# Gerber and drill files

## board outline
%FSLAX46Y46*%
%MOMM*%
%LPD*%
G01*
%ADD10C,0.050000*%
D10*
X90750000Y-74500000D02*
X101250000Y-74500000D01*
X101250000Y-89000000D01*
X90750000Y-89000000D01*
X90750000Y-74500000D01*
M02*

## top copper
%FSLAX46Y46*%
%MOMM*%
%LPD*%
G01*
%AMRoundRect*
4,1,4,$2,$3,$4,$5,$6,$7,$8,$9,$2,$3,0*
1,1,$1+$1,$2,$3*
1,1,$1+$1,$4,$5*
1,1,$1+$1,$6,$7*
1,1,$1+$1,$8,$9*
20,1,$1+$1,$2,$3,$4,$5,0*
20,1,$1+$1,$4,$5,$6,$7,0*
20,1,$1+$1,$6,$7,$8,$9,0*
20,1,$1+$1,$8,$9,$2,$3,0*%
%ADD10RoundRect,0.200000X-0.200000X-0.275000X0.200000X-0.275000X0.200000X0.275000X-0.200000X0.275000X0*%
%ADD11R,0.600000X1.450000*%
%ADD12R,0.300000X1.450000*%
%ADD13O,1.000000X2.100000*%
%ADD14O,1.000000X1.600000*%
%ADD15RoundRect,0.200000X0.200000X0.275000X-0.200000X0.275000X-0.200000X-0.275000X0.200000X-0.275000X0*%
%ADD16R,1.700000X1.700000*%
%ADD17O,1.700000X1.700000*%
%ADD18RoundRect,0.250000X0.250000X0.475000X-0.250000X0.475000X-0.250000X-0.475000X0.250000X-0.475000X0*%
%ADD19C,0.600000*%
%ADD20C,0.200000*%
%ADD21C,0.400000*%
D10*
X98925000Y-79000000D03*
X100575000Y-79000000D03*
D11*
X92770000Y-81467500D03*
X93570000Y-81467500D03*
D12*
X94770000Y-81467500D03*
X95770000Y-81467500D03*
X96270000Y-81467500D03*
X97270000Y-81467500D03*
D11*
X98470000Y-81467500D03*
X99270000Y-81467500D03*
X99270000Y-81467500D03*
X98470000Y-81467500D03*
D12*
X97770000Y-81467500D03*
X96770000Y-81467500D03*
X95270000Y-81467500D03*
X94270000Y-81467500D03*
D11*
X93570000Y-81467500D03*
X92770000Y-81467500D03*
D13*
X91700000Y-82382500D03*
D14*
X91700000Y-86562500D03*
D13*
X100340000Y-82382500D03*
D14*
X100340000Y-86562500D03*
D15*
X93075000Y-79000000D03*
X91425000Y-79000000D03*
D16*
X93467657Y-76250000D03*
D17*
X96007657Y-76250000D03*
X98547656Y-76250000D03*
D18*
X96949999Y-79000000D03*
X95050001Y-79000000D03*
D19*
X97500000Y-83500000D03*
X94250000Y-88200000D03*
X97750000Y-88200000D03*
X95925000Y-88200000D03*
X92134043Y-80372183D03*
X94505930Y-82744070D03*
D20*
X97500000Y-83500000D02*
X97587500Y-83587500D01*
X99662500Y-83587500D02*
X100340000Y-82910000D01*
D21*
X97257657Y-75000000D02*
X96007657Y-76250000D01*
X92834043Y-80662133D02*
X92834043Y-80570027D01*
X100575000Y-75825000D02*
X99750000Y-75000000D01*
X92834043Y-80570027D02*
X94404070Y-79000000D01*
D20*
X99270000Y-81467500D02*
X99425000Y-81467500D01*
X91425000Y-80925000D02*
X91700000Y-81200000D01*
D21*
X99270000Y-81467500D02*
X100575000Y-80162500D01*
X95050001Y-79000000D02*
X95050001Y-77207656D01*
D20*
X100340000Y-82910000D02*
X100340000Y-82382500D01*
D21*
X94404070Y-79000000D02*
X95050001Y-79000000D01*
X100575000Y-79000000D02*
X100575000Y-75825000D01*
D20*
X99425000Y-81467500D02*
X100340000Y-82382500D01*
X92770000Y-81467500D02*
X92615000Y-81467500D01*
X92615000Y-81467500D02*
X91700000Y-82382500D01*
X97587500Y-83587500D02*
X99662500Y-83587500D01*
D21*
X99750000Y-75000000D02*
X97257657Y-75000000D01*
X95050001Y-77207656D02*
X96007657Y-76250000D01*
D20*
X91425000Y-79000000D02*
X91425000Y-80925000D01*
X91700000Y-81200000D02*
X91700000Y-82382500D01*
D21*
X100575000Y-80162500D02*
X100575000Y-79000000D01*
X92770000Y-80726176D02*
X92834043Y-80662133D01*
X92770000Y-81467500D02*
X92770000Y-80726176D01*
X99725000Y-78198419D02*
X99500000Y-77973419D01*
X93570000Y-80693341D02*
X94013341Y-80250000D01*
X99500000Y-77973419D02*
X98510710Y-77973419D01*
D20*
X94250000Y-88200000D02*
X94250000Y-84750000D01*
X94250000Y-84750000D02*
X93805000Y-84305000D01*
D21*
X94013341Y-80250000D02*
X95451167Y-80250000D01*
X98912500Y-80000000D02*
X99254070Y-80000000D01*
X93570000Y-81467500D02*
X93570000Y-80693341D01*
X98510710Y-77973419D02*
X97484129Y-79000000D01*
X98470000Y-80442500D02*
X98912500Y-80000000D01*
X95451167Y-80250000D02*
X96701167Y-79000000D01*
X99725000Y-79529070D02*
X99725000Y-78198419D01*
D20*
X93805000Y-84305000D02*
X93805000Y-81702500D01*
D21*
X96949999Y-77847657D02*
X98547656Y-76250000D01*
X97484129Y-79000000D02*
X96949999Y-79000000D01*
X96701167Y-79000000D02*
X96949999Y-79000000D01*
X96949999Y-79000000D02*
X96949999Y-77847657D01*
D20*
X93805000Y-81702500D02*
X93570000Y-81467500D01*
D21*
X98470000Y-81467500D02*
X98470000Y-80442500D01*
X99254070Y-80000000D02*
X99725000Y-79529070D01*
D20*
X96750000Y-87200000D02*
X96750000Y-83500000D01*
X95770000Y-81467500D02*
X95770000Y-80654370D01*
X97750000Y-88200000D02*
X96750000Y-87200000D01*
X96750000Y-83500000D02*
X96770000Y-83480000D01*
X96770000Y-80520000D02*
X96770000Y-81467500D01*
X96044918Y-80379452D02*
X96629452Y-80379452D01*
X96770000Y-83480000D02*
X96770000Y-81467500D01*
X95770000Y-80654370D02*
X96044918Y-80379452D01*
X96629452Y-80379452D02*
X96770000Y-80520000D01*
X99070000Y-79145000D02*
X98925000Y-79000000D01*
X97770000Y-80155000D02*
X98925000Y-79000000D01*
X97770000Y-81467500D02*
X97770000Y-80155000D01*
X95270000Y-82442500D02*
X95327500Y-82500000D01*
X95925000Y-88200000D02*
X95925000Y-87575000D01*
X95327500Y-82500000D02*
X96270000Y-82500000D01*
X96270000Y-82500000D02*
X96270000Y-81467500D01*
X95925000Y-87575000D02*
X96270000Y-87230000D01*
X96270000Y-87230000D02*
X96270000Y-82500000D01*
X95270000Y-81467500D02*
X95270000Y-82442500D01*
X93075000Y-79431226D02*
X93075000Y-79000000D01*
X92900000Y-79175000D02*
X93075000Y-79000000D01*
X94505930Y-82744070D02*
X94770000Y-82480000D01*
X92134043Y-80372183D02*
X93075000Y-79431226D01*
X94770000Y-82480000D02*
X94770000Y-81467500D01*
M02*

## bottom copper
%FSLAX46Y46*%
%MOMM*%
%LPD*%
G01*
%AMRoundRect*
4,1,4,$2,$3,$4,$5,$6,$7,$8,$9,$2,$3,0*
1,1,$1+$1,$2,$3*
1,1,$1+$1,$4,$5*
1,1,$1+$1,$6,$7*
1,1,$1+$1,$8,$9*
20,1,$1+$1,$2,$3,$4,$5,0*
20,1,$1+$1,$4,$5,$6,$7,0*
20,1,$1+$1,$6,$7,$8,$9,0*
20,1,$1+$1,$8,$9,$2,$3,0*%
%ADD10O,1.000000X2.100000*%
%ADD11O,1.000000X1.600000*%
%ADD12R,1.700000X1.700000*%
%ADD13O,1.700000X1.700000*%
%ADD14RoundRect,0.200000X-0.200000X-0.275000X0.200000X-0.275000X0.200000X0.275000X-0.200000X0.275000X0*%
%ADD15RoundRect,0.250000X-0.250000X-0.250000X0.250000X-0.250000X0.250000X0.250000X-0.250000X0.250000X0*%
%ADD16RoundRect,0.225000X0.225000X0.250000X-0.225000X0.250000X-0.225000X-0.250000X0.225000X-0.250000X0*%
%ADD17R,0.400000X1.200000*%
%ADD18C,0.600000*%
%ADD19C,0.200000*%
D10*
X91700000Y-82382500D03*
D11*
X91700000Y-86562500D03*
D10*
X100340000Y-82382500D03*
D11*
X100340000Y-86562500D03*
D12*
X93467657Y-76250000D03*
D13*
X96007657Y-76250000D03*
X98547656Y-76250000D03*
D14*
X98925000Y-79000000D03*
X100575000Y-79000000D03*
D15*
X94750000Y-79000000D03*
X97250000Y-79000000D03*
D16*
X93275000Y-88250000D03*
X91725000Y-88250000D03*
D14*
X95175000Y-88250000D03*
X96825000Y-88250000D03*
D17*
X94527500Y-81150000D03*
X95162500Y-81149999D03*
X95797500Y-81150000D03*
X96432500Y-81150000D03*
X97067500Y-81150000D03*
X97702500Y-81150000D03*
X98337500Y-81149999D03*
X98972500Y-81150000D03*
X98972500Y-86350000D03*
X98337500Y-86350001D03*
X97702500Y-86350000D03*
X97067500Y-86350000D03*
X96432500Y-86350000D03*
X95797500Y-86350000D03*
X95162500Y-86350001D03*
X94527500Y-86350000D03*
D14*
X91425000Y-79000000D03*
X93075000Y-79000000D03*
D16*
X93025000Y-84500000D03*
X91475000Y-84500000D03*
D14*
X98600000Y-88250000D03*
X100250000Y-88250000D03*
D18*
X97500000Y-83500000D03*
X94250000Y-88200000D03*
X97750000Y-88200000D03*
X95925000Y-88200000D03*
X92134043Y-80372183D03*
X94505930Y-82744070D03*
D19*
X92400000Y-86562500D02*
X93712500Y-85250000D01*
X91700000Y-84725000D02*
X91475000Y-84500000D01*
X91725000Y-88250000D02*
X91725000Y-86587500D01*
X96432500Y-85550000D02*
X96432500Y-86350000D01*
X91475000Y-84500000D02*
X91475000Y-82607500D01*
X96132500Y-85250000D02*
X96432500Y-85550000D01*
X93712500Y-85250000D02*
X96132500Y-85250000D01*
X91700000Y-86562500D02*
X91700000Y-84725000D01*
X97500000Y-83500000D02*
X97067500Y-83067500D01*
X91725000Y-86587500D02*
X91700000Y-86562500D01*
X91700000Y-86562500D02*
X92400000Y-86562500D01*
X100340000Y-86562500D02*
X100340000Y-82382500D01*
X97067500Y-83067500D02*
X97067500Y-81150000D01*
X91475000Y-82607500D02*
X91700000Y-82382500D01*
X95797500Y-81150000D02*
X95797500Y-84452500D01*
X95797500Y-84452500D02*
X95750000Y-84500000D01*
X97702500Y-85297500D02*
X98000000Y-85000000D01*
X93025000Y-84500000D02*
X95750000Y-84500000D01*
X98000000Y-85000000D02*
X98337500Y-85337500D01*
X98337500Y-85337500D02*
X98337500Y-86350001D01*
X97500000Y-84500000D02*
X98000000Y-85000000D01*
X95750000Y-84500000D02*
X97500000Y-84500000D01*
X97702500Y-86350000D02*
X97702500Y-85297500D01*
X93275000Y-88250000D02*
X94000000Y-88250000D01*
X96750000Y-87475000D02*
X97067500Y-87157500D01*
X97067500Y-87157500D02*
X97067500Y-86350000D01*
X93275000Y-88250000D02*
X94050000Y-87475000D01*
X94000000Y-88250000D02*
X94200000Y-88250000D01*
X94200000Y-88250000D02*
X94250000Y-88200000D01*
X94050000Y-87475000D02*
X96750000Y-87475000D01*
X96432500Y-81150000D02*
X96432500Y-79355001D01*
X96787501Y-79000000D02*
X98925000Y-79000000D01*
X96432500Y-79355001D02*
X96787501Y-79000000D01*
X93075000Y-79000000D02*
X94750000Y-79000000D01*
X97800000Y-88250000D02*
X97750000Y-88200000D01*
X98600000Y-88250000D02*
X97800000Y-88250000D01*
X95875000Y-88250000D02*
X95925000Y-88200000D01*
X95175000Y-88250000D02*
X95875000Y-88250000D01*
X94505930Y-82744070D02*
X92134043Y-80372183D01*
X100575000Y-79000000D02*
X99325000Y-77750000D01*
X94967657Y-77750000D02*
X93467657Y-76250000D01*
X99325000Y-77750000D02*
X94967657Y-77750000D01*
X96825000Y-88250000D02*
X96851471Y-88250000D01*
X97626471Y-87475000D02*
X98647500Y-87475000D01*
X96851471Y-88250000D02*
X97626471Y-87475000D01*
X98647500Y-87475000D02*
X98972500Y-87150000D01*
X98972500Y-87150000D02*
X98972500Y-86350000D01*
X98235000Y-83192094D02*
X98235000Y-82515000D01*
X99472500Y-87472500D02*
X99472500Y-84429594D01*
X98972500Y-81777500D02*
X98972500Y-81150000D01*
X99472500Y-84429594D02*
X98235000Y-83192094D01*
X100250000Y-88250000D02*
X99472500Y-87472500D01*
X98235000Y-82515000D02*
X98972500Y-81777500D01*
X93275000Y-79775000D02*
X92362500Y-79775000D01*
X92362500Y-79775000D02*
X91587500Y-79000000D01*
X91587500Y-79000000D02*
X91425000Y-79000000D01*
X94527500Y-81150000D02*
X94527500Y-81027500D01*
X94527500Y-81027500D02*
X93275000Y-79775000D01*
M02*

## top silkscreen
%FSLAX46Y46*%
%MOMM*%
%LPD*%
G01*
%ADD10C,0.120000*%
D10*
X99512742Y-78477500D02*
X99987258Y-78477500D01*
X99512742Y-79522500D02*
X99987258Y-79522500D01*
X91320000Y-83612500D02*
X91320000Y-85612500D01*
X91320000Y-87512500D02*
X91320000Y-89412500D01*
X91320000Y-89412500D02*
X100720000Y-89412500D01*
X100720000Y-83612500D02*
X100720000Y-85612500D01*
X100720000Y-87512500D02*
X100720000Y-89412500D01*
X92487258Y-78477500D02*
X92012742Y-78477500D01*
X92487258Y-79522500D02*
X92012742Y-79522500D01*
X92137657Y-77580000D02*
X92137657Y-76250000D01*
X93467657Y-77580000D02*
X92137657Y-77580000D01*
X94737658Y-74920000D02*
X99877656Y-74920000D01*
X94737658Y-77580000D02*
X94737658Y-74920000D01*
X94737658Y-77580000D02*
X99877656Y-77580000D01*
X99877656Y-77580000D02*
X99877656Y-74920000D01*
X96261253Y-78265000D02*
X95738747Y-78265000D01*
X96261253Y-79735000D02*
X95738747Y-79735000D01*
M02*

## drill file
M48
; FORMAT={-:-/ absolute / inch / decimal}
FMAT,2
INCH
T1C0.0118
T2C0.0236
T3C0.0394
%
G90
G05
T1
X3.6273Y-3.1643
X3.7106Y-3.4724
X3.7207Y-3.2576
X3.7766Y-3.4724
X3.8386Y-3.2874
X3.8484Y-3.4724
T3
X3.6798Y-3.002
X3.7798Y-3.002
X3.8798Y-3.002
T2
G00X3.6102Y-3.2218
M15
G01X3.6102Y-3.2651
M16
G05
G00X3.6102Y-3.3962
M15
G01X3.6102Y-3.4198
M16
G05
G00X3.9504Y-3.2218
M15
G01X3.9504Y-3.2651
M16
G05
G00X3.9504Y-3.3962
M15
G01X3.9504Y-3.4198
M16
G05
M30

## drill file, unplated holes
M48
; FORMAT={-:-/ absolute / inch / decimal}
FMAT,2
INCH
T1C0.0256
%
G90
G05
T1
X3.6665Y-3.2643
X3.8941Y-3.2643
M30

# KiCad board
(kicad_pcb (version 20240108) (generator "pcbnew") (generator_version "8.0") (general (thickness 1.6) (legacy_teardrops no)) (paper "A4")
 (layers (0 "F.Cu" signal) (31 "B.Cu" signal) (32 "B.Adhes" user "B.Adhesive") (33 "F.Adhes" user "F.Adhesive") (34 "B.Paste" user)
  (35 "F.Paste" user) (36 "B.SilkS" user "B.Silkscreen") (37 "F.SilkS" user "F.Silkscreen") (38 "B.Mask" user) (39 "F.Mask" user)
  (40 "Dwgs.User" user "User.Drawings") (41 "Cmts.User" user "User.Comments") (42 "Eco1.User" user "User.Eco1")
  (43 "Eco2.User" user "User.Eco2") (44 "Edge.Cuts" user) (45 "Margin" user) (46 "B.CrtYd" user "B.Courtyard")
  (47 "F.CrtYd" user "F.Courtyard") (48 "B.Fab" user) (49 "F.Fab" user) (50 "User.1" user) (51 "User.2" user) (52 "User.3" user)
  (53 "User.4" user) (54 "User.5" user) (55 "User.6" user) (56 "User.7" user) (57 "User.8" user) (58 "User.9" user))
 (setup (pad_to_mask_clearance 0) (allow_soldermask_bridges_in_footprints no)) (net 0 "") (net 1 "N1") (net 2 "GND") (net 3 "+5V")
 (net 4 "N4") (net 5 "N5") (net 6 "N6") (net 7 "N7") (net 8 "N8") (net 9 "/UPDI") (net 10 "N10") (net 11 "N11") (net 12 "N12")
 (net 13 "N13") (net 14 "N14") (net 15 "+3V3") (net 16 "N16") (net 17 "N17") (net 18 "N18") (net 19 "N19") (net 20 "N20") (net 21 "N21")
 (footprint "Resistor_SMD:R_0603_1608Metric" (layer "F.Cu") (at 99.75 79)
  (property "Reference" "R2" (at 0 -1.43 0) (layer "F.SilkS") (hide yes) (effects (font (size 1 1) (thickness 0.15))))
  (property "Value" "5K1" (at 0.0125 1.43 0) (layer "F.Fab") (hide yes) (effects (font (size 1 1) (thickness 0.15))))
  (fp_line (start -0.237258 -0.5225) (end 0.237258 -0.5225) (stroke (width 0.12) (type solid)) (layer "F.SilkS"))
  (fp_line (start -0.237258 0.5225) (end 0.237258 0.5225) (stroke (width 0.12) (type solid)) (layer "F.SilkS"))
  (pad "1" smd roundrect (at -0.825 0) (size 0.8 0.95) (layers "F.Cu" "F.Paste" "F.Mask") (roundrect_rratio 0.25) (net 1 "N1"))
  (pad "2" smd roundrect (at 0.825 0) (size 0.8 0.95) (layers "F.Cu" "F.Paste" "F.Mask") (roundrect_rratio 0.25) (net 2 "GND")))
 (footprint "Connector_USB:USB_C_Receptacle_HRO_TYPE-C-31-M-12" (layer "F.Cu") (at 96.02 85.5125)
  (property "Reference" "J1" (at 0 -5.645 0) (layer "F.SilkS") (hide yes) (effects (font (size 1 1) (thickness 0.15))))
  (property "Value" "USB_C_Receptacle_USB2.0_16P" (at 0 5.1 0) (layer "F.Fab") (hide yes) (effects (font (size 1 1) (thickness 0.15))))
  (fp_line (start -4.7 -1.9) (end -4.7 0.1) (stroke (width 0.12) (type solid)) (layer "F.SilkS"))
  (fp_line (start -4.7 2) (end -4.7 3.9) (stroke (width 0.12) (type solid)) (layer "F.SilkS"))
  (fp_line (start -4.7 3.9) (end 4.7 3.9) (stroke (width 0.12) (type solid)) (layer "F.SilkS"))
  (fp_line (start 4.7 -1.9) (end 4.7 0.1) (stroke (width 0.12) (type solid)) (layer "F.SilkS"))
  (fp_line (start 4.7 2) (end 4.7 3.9) (stroke (width 0.12) (type solid)) (layer "F.SilkS"))
  (pad "" np_thru_hole circle (at -2.89 -2.6) (size 0.65 0.65) (drill 0.65) (layers "*.Cu" "*.Mask"))
  (pad "" np_thru_hole circle (at 2.89 -2.6) (size 0.65 0.65) (drill 0.65) (layers "*.Cu" "*.Mask"))
  (pad "A1" smd rect (at -3.25 -4.045) (size 0.6 1.45) (layers "F.Cu" "F.Paste" "F.Mask") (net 2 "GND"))
  (pad "A4" smd rect (at -2.45 -4.045) (size 0.6 1.45) (layers "F.Cu" "F.Paste" "F.Mask") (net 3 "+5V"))
  (pad "A5" smd rect (at -1.25 -4.045) (size 0.3 1.45) (layers "F.Cu" "F.Paste" "F.Mask") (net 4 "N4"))
  (pad "A6" smd rect (at -0.25 -4.045) (size 0.3 1.45) (layers "F.Cu" "F.Paste" "F.Mask") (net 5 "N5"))
  (pad "A7" smd rect (at 0.25 -4.045) (size 0.3 1.45) (layers "F.Cu" "F.Paste" "F.Mask") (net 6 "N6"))
  (pad "A8" smd rect (at 1.25 -4.045) (size 0.3 1.45) (layers "F.Cu" "F.Paste" "F.Mask") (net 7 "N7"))
  (pad "A9" smd rect (at 2.45 -4.045) (size 0.6 1.45) (layers "F.Cu" "F.Paste" "F.Mask") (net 3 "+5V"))
  (pad "A12" smd rect (at 3.25 -4.045) (size 0.6 1.45) (layers "F.Cu" "F.Paste" "F.Mask") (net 2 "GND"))
  (pad "B1" smd rect (at 3.25 -4.045) (size 0.6 1.45) (layers "F.Cu" "F.Paste" "F.Mask") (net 2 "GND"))
  (pad "B4" smd rect (at 2.45 -4.045) (size 0.6 1.45) (layers "F.Cu" "F.Paste" "F.Mask") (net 3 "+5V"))
  (pad "B5" smd rect (at 1.75 -4.045) (size 0.3 1.45) (layers "F.Cu" "F.Paste" "F.Mask") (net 1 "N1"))
  (pad "B6" smd rect (at 0.75 -4.045) (size 0.3 1.45) (layers "F.Cu" "F.Paste" "F.Mask") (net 5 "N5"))
  (pad "B7" smd rect (at -0.75 -4.045) (size 0.3 1.45) (layers "F.Cu" "F.Paste" "F.Mask") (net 6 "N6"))
  (pad "B8" smd rect (at -1.75 -4.045) (size 0.3 1.45) (layers "F.Cu" "F.Paste" "F.Mask") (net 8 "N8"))
  (pad "B9" smd rect (at -2.45 -4.045) (size 0.6 1.45) (layers "F.Cu" "F.Paste" "F.Mask") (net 3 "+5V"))
  (pad "B12" smd rect (at -3.25 -4.045) (size 0.6 1.45) (layers "F.Cu" "F.Paste" "F.Mask") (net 2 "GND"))
  (pad "S1" thru_hole oval (at -4.32 -3.13) (size 1 2.1) (drill oval 0.6 1.7) (layers "*.Cu" "*.Mask") (remove_unused_layers no)
   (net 2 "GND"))
  (pad "S1" thru_hole oval (at -4.32 1.05) (size 1 1.6) (drill oval 0.6 1.2) (layers "*.Cu" "*.Mask") (remove_unused_layers no)
   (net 2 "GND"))
  (pad "S1" thru_hole oval (at 4.32 -3.13) (size 1 2.1) (drill oval 0.6 1.7) (layers "*.Cu" "*.Mask") (remove_unused_layers no)
   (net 2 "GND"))
  (pad "S1" thru_hole oval (at 4.32 1.05) (size 1 1.6) (drill oval 0.6 1.2) (layers "*.Cu" "*.Mask") (remove_unused_layers no) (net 2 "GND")))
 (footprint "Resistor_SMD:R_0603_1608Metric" (layer "F.Cu") (at 92.25 79 180)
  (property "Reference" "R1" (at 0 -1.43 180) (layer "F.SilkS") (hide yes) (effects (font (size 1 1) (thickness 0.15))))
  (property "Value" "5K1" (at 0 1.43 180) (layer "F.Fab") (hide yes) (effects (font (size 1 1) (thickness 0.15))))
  (fp_line (start -0.237258 0.5225) (end 0.237258 0.5225) (stroke (width 0.12) (type solid)) (layer "F.SilkS"))
  (fp_line (start -0.237258 -0.5225) (end 0.237258 -0.5225) (stroke (width 0.12) (type solid)) (layer "F.SilkS"))
  (pad "1" smd roundrect (at -0.825 0 180) (size 0.8 0.95) (layers "F.Cu" "F.Paste" "F.Mask") (roundrect_rratio 0.25) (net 4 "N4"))
  (pad "2" smd roundrect (at 0.825 0 180) (size 0.8 0.95) (layers "F.Cu" "F.Paste" "F.Mask") (roundrect_rratio 0.25) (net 2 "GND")))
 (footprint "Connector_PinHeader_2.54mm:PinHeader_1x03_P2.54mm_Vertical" (layer "F.Cu") (at 93.467657 76.25 90)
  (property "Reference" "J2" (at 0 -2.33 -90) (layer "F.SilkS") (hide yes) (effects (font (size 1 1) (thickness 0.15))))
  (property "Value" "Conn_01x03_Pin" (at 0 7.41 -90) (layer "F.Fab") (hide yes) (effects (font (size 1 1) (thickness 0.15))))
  (fp_line (start -1.33 -1.33) (end 0 -1.33) (stroke (width 0.12) (type solid)) (layer "F.SilkS"))
  (fp_line (start -1.33 0) (end -1.33 -1.33) (stroke (width 0.12) (type solid)) (layer "F.SilkS"))
  (fp_line (start 1.33 1.270001) (end 1.33 6.409999) (stroke (width 0.12) (type solid)) (layer "F.SilkS"))
  (fp_line (start -1.33 1.270001) (end 1.33 1.270001) (stroke (width 0.12) (type solid)) (layer "F.SilkS"))
  (fp_line (start -1.33 1.270001) (end -1.33 6.409999) (stroke (width 0.12) (type solid)) (layer "F.SilkS"))
  (fp_line (start -1.33 6.409999) (end 1.33 6.409999) (stroke (width 0.12) (type solid)) (layer "F.SilkS"))
  (pad "1" thru_hole rect (at 0 0 90) (size 1.7 1.7) (drill 1) (layers "*.Cu" "*.Mask") (remove_unused_layers no) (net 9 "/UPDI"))
  (pad "2" thru_hole oval (at 0 2.54 90) (size 1.7 1.7) (drill 1) (layers "*.Cu" "*.Mask") (remove_unused_layers no) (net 2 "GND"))
  (pad "3" thru_hole oval (at 0 5.079999 90) (size 1.7 1.7) (drill 1) (layers "*.Cu" "*.Mask") (remove_unused_layers no) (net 3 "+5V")))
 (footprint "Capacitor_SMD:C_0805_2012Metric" (layer "F.Cu") (at 96 79 180)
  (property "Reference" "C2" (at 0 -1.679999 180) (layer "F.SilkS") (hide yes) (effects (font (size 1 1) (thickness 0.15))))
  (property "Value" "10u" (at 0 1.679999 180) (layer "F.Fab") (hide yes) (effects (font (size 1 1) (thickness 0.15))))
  (fp_line (start -0.261253 0.735) (end 0.261253 0.735) (stroke (width 0.12) (type solid)) (layer "F.SilkS"))
  (fp_line (start -0.261253 -0.735) (end 0.261253 -0.735) (stroke (width 0.12) (type solid)) (layer "F.SilkS"))
  (pad "1" smd roundrect (at -0.949999 0 180) (size 1 1.45) (layers "F.Cu" "F.Paste" "F.Mask") (roundrect_rratio 0.25) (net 3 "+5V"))
  (pad "2" smd roundrect (at 0.949999 0 180) (size 1 1.45) (layers "F.Cu" "F.Paste" "F.Mask") (roundrect_rratio 0.25) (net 2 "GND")))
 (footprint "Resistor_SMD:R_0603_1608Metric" (layer "B.Cu") (at 99.75 79)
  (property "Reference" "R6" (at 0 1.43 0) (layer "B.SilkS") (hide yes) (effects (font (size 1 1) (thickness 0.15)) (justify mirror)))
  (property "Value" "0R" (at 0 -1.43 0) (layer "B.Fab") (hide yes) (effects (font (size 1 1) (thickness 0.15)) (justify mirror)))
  (pad "1" smd roundrect (at -0.825 0) (size 0.8 0.95) (layers "B.Cu" "B.Paste" "B.Mask") (roundrect_rratio 0.25) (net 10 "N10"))
  (pad "2" smd roundrect (at 0.825 0) (size 0.8 0.95) (layers "B.Cu" "B.Paste" "B.Mask") (roundrect_rratio 0.25) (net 9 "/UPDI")))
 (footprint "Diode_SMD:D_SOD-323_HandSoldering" (layer "B.Cu") (at 96 79)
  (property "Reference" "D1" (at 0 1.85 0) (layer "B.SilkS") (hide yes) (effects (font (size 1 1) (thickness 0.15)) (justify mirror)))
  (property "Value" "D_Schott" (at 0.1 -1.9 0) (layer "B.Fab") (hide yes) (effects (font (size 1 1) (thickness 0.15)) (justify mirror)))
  (pad "1" smd roundrect (at -1.25 0) (size 1 1) (layers "B.Cu" "B.Paste" "B.Mask") (roundrect_rratio 0.25) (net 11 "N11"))
  (pad "2" smd roundrect (at 1.25 0) (size 1 1) (layers "B.Cu" "B.Paste" "B.Mask") (roundrect_rratio 0.25) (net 10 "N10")))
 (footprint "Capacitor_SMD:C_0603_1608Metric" (layer "B.Cu") (at 92.5 88.25 180)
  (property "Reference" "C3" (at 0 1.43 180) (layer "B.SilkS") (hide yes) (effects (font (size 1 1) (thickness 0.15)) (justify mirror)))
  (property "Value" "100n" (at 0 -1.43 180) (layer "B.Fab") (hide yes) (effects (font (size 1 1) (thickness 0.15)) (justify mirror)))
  (pad "1" smd roundrect (at -0.775 0 180) (size 0.9 0.95) (layers "B.Cu" "B.Paste" "B.Mask") (roundrect_rratio 0.25) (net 3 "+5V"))
  (pad "2" smd roundrect (at 0.775 0 180) (size 0.9 0.95) (layers "B.Cu" "B.Paste" "B.Mask") (roundrect_rratio 0.25) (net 2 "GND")))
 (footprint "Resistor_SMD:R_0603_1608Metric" (layer "B.Cu") (at 96 88.25)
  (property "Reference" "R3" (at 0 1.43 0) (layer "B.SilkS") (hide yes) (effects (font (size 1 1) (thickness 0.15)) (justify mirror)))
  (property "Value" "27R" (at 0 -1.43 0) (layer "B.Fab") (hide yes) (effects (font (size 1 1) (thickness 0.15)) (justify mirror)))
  (pad "1" smd roundrect (at -0.825 0) (size 0.8 0.95) (layers "B.Cu" "B.Paste" "B.Mask") (roundrect_rratio 0.25) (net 6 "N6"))
  (pad "2" smd roundrect (at 0.825 0) (size 0.8 0.95) (layers "B.Cu" "B.Paste" "B.Mask") (roundrect_rratio 0.25) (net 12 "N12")))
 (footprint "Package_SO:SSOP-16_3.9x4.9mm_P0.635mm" (layer "B.Cu") (at 96.75 83.75 -90)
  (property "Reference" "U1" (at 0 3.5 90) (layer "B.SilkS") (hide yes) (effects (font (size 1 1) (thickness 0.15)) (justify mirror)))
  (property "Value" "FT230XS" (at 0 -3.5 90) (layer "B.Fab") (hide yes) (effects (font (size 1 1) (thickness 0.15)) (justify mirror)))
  (pad "1" smd rect (at -2.6 2.2225 270) (size 1.2 0.4) (layers "B.Cu" "B.Paste" "B.Mask") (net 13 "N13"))
  (pad "2" smd rect (at -2.600001 1.5875 270) (size 1.2 0.4) (layers "B.Cu" "B.Paste" "B.Mask") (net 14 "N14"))
  (pad "3" smd rect (at -2.6 0.9525 270) (size 1.2 0.4) (layers "B.Cu" "B.Paste" "B.Mask") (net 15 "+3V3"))
  (pad "4" smd rect (at -2.6 0.3175 270) (size 1.2 0.4) (layers "B.Cu" "B.Paste" "B.Mask") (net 10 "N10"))
  (pad "5" smd rect (at -2.6 -0.3175 270) (size 1.2 0.4) (layers "B.Cu" "B.Paste" "B.Mask") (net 2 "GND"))
  (pad "6" smd rect (at -2.6 -0.9525 270) (size 1.2 0.4) (layers "B.Cu" "B.Paste" "B.Mask") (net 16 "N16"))
  (pad "7" smd rect (at -2.600001 -1.5875 270) (size 1.2 0.4) (layers "B.Cu" "B.Paste" "B.Mask") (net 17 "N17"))
  (pad "8" smd rect (at -2.6 -2.2225 270) (size 1.2 0.4) (layers "B.Cu" "B.Paste" "B.Mask") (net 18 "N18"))
  (pad "9" smd rect (at 2.6 -2.2225 270) (size 1.2 0.4) (layers "B.Cu" "B.Paste" "B.Mask") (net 12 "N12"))
  (pad "10" smd rect (at 2.600001 -1.5875 270) (size 1.2 0.4) (layers "B.Cu" "B.Paste" "B.Mask") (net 15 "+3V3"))
  (pad "11" smd rect (at 2.6 -0.9525 270) (size 1.2 0.4) (layers "B.Cu" "B.Paste" "B.Mask") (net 15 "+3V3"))
  (pad "12" smd rect (at 2.6 -0.3175 270) (size 1.2 0.4) (layers "B.Cu" "B.Paste" "B.Mask") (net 3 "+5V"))
  (pad "13" smd rect (at 2.6 0.3175 270) (size 1.2 0.4) (layers "B.Cu" "B.Paste" "B.Mask") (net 2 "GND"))
  (pad "14" smd rect (at 2.6 0.9525 270) (size 1.2 0.4) (layers "B.Cu" "B.Paste" "B.Mask") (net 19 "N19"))
  (pad "15" smd rect (at 2.600001 1.5875 270) (size 1.2 0.4) (layers "B.Cu" "B.Paste" "B.Mask") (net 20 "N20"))
  (pad "16" smd rect (at 2.6 2.2225 270) (size 1.2 0.4) (layers "B.Cu" "B.Paste" "B.Mask") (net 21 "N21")))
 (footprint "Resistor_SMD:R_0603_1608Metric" (layer "B.Cu") (at 92.25 79)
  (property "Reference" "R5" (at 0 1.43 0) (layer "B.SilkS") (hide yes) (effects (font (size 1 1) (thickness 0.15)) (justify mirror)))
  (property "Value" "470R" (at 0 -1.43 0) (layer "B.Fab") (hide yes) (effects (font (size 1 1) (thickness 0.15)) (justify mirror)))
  (pad "1" smd roundrect (at -0.825 0) (size 0.8 0.95) (layers "B.Cu" "B.Paste" "B.Mask") (roundrect_rratio 0.25) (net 13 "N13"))
  (pad "2" smd roundrect (at 0.825 0) (size 0.8 0.95) (layers "B.Cu" "B.Paste" "B.Mask") (roundrect_rratio 0.25) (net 11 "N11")))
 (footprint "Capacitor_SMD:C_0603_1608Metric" (layer "B.Cu") (at 92.25 84.5 180)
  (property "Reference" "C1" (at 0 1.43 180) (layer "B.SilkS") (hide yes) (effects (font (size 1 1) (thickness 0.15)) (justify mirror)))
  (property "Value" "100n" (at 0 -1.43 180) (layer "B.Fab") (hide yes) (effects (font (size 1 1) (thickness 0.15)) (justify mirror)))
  (pad "1" smd roundrect (at -0.775 0 180) (size 0.9 0.95) (layers "B.Cu" "B.Paste" "B.Mask") (roundrect_rratio 0.25) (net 15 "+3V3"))
  (pad "2" smd roundrect (at 0.775 0 180) (size 0.9 0.95) (layers "B.Cu" "B.Paste" "B.Mask") (roundrect_rratio 0.25) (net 2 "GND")))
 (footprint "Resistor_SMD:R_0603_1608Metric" (layer "B.Cu") (at 99.425 88.25)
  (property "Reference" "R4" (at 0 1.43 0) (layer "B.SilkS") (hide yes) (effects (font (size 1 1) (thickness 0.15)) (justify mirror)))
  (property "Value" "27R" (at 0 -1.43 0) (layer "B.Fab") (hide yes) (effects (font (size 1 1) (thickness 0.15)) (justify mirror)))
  (pad "1" smd roundrect (at -0.825 0) (size 0.8 0.95) (layers "B.Cu" "B.Paste" "B.Mask") (roundrect_rratio 0.25) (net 5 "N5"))
  (pad "2" smd roundrect (at 0.825 0) (size 0.8 0.95) (layers "B.Cu" "B.Paste" "B.Mask") (roundrect_rratio 0.25) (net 18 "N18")))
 (gr_rect (start 90.75 74.5) (end 101.25 89) (stroke (width 0.05) (type default)) (fill none) (layer "Edge.Cuts"))
 (segment (start 97.5 83.5) (end 97.5875 83.5875) (width 0.2) (layer "F.Cu") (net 2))
 (segment (start 99.6625 83.5875) (end 100.34 82.91) (width 0.2) (layer "F.Cu") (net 2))
 (segment (start 97.257657 75) (end 96.007657 76.25) (width 0.4) (layer "F.Cu") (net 2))
 (segment (start 92.834043 80.662133) (end 92.834043 80.570027) (width 0.4) (layer "F.Cu") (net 2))
 (segment (start 100.575 75.825) (end 99.75 75) (width 0.4) (layer "F.Cu") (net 2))
 (segment (start 92.834043 80.570027) (end 94.40407 79) (width 0.4) (layer "F.Cu") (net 2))
 (segment (start 99.27 81.4675) (end 99.425 81.4675) (width 0.2) (layer "F.Cu") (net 2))
 (segment (start 91.425 80.925) (end 91.7 81.2) (width 0.2) (layer "F.Cu") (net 2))
 (segment (start 99.27 81.4675) (end 100.575 80.1625) (width 0.4) (layer "F.Cu") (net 2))
 (segment (start 95.050001 79) (end 95.050001 77.207656) (width 0.4) (layer "F.Cu") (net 2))
 (segment (start 100.34 82.91) (end 100.34 82.3825) (width 0.2) (layer "F.Cu") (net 2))
 (segment (start 94.40407 79) (end 95.050001 79) (width 0.4) (layer "F.Cu") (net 2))
 (segment (start 100.575 79) (end 100.575 75.825) (width 0.4) (layer "F.Cu") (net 2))
 (segment (start 99.425 81.4675) (end 100.34 82.3825) (width 0.2) (layer "F.Cu") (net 2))
 (segment (start 92.77 81.4675) (end 92.615 81.4675) (width 0.2) (layer "F.Cu") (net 2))
 (segment (start 92.615 81.4675) (end 91.7 82.3825) (width 0.2) (layer "F.Cu") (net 2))
 (segment (start 97.5875 83.5875) (end 99.6625 83.5875) (width 0.2) (layer "F.Cu") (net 2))
 (segment (start 99.75 75) (end 97.257657 75) (width 0.4) (layer "F.Cu") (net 2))
 (segment (start 95.050001 77.207656) (end 96.007657 76.25) (width 0.4) (layer "F.Cu") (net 2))
 (segment (start 91.425 79) (end 91.425 80.925) (width 0.2) (layer "F.Cu") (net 2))
 (segment (start 91.7 81.2) (end 91.7 82.3825) (width 0.2) (layer "F.Cu") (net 2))
 (segment (start 100.575 80.1625) (end 100.575 79) (width 0.4) (layer "F.Cu") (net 2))
 (segment (start 92.77 80.726176) (end 92.834043 80.662133) (width 0.4) (layer "F.Cu") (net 2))
 (segment (start 92.77 81.4675) (end 92.77 80.726176) (width 0.4) (layer "F.Cu") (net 2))
 (via (at 97.5 83.5) (size 0.6) (drill 0.3) (layers "F.Cu" "B.Cu") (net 2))
 (segment (start 92.4 86.5625) (end 93.7125 85.25) (width 0.2) (layer "B.Cu") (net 2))
 (segment (start 91.7 84.725) (end 91.475 84.5) (width 0.2) (layer "B.Cu") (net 2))
 (segment (start 91.725 88.25) (end 91.725 86.5875) (width 0.2) (layer "B.Cu") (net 2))
 (segment (start 96.4325 85.55) (end 96.4325 86.35) (width 0.2) (layer "B.Cu") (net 2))
 (segment (start 91.475 84.5) (end 91.475 82.6075) (width 0.2) (layer "B.Cu") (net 2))
 (segment (start 96.1325 85.25) (end 96.4325 85.55) (width 0.2) (layer "B.Cu") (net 2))
 (segment (start 93.7125 85.25) (end 96.1325 85.25) (width 0.2) (layer "B.Cu") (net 2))
 (segment (start 91.7 86.5625) (end 91.7 84.725) (width 0.2) (layer "B.Cu") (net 2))
 (segment (start 97.5 83.5) (end 97.0675 83.0675) (width 0.2) (layer "B.Cu") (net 2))
 (segment (start 91.725 86.5875) (end 91.7 86.5625) (width 0.2) (layer "B.Cu") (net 2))
 (segment (start 91.7 86.5625) (end 92.4 86.5625) (width 0.2) (layer "B.Cu") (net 2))
 (segment (start 100.34 86.5625) (end 100.34 82.3825) (width 0.2) (layer "B.Cu") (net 2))
 (segment (start 97.0675 83.0675) (end 97.0675 81.15) (width 0.2) (layer "B.Cu") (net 2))
 (segment (start 91.475 82.6075) (end 91.7 82.3825) (width 0.2) (layer "B.Cu") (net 2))
 (segment (start 95.7975 81.15) (end 95.7975 84.4525) (width 0.2) (layer "B.Cu") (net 15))
 (segment (start 95.7975 84.4525) (end 95.75 84.5) (width 0.2) (layer "B.Cu") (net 15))
 (segment (start 97.7025 85.2975) (end 98 85) (width 0.2) (layer "B.Cu") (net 15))
 (segment (start 93.025 84.5) (end 95.75 84.5) (width 0.2) (layer "B.Cu") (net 15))
 (segment (start 98 85) (end 98.3375 85.3375) (width 0.2) (layer "B.Cu") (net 15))
 (segment (start 98.3375 85.3375) (end 98.3375 86.350001) (width 0.2) (layer "B.Cu") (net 15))
 (segment (start 97.5 84.5) (end 98 85) (width 0.2) (layer "B.Cu") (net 15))
 (segment (start 95.75 84.5) (end 97.5 84.5) (width 0.2) (layer "B.Cu") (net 15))
 (segment (start 97.7025 86.35) (end 97.7025 85.2975) (width 0.2) (layer "B.Cu") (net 15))
 (segment (start 99.725 78.198419) (end 99.5 77.973419) (width 0.4) (layer "F.Cu") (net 3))
 (segment (start 93.57 80.693341) (end 94.013341 80.25) (width 0.4) (layer "F.Cu") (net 3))
 (segment (start 99.5 77.973419) (end 98.51071 77.973419) (width 0.4) (layer "F.Cu") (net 3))
 (segment (start 94.25 88.2) (end 94.25 84.75) (width 0.2) (layer "F.Cu") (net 3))
 (segment (start 94.25 84.75) (end 93.805 84.305) (width 0.2) (layer "F.Cu") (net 3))
 (segment (start 94.013341 80.25) (end 95.451167 80.25) (width 0.4) (layer "F.Cu") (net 3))
 (segment (start 98.9125 80) (end 99.25407 80) (width 0.4) (layer "F.Cu") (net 3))
 (segment (start 93.57 81.4675) (end 93.57 80.693341) (width 0.4) (layer "F.Cu") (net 3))
 (segment (start 98.51071 77.973419) (end 97.484129 79) (width 0.4) (layer "F.Cu") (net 3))
 (segment (start 98.47 80.4425) (end 98.9125 80) (width 0.4) (layer "F.Cu") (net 3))
 (segment (start 95.451167 80.25) (end 96.701167 79) (width 0.4) (layer "F.Cu") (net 3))
 (segment (start 99.725 79.52907) (end 99.725 78.198419) (width 0.4) (layer "F.Cu") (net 3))
 (segment (start 93.805 84.305) (end 93.805 81.7025) (width 0.2) (layer "F.Cu") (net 3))
 (segment (start 96.949999 77.847657) (end 98.547656 76.25) (width 0.4) (layer "F.Cu") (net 3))
 (segment (start 97.484129 79) (end 96.949999 79) (width 0.4) (layer "F.Cu") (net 3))
 (segment (start 96.701167 79) (end 96.949999 79) (width 0.4) (layer "F.Cu") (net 3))
 (segment (start 96.949999 79) (end 96.949999 77.847657) (width 0.4) (layer "F.Cu") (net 3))
 (segment (start 93.805 81.7025) (end 93.57 81.4675) (width 0.2) (layer "F.Cu") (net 3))
 (segment (start 98.47 81.4675) (end 98.47 80.4425) (width 0.4) (layer "F.Cu") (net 3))
 (segment (start 99.25407 80) (end 99.725 79.52907) (width 0.4) (layer "F.Cu") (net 3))
 (via (at 94.25 88.2) (size 0.6) (drill 0.3) (layers "F.Cu" "B.Cu") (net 3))
 (segment (start 93.275 88.25) (end 94 88.25) (width 0.2) (layer "B.Cu") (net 3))
 (segment (start 96.75 87.475) (end 97.0675 87.1575) (width 0.2) (layer "B.Cu") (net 3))
 (segment (start 97.0675 87.1575) (end 97.0675 86.35) (width 0.2) (layer "B.Cu") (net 3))
 (segment (start 93.275 88.25) (end 94.05 87.475) (width 0.2) (layer "B.Cu") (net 3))
 (segment (start 94 88.25) (end 94.2 88.25) (width 0.2) (layer "B.Cu") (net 3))
 (segment (start 94.2 88.25) (end 94.25 88.2) (width 0.2) (layer "B.Cu") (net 3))
 (segment (start 94.05 87.475) (end 96.75 87.475) (width 0.2) (layer "B.Cu") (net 3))
 (segment (start 96.4325 81.15) (end 96.4325 79.355001) (width 0.2) (layer "B.Cu") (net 10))
 (segment (start 96.787501 79) (end 98.925 79) (width 0.2) (layer "B.Cu") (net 10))
 (segment (start 96.4325 79.355001) (end 96.787501 79) (width 0.2) (layer "B.Cu") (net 10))
 (segment (start 93.075 79) (end 94.75 79) (width 0.2) (layer "B.Cu") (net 11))
 (segment (start 96.75 87.2) (end 96.75 83.5) (width 0.2) (layer "F.Cu") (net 5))
 (segment (start 95.77 81.4675) (end 95.77 80.65437) (width 0.2) (layer "F.Cu") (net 5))
 (segment (start 97.75 88.2) (end 96.75 87.2) (width 0.2) (layer "F.Cu") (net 5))
 (segment (start 96.75 83.5) (end 96.77 83.48) (width 0.2) (layer "F.Cu") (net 5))
 (segment (start 96.77 80.52) (end 96.77 81.4675) (width 0.2) (layer "F.Cu") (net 5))
 (segment (start 96.044918 80.379452) (end 96.629452 80.379452) (width 0.2) (layer "F.Cu") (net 5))
 (segment (start 96.77 83.48) (end 96.77 81.4675) (width 0.2) (layer "F.Cu") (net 5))
 (segment (start 95.77 80.65437) (end 96.044918 80.379452) (width 0.2) (layer "F.Cu") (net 5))
 (segment (start 96.629452 80.379452) (end 96.77 80.52) (width 0.2) (layer "F.Cu") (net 5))
 (via (at 97.75 88.2) (size 0.6) (drill 0.3) (layers "F.Cu" "B.Cu") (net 5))
 (segment (start 97.8 88.25) (end 97.75 88.2) (width 0.2) (layer "B.Cu") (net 5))
 (segment (start 98.6 88.25) (end 97.8 88.25) (width 0.2) (layer "B.Cu") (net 5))
 (segment (start 99.07 79.145) (end 98.925 79) (width 0.2) (layer "F.Cu") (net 1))
 (segment (start 97.77 80.155) (end 98.925 79) (width 0.2) (layer "F.Cu") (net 1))
 (segment (start 97.77 81.4675) (end 97.77 80.155) (width 0.2) (layer "F.Cu") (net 1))
 (segment (start 95.27 82.4425) (end 95.3275 82.5) (width 0.2) (layer "F.Cu") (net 6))
 (segment (start 95.925 88.2) (end 95.925 87.575) (width 0.2) (layer "F.Cu") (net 6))
 (segment (start 95.3275 82.5) (end 96.27 82.5) (width 0.2) (layer "F.Cu") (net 6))
 (segment (start 96.27 82.5) (end 96.27 81.4675) (width 0.2) (layer "F.Cu") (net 6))
 (segment (start 95.925 87.575) (end 96.27 87.23) (width 0.2) (layer "F.Cu") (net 6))
 (segment (start 96.27 87.23) (end 96.27 82.5) (width 0.2) (layer "F.Cu") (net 6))
 (segment (start 95.27 81.4675) (end 95.27 82.4425) (width 0.2) (layer "F.Cu") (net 6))
 (via (at 95.925 88.2) (size 0.6) (drill 0.3) (layers "F.Cu" "B.Cu") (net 6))
 (segment (start 95.875 88.25) (end 95.925 88.2) (width 0.2) (layer "B.Cu") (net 6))
 (segment (start 95.175 88.25) (end 95.875 88.25) (width 0.2) (layer "B.Cu") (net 6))
 (segment (start 93.075 79.431226) (end 93.075 79) (width 0.2) (layer "F.Cu") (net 4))
 (segment (start 92.9 79.175) (end 93.075 79) (width 0.2) (layer "F.Cu") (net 4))
 (segment (start 94.50593 82.74407) (end 94.77 82.48) (width 0.2) (layer "F.Cu") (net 4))
 (segment (start 92.134043 80.372183) (end 93.075 79.431226) (width 0.2) (layer "F.Cu") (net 4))
 (segment (start 94.77 82.48) (end 94.77 81.4675) (width 0.2) (layer "F.Cu") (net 4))
 (via (at 92.134043 80.372183) (size 0.6) (drill 0.3) (layers "F.Cu" "B.Cu") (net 4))
 (via (at 94.50593 82.74407) (size 0.6) (drill 0.3) (layers "F.Cu" "B.Cu") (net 4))
 (segment (start 94.50593 82.74407) (end 92.134043 80.372183) (width 0.2) (layer "B.Cu") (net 4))
 (segment (start 100.575 79) (end 99.325 77.75) (width 0.2) (layer "B.Cu") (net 9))
 (segment (start 94.967657 77.75) (end 93.467657 76.25) (width 0.2) (layer "B.Cu") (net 9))
 (segment (start 99.325 77.75) (end 94.967657 77.75) (width 0.2) (layer "B.Cu") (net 9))
 (segment (start 96.825 88.25) (end 96.851471 88.25) (width 0.2) (layer "B.Cu") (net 12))
 (segment (start 97.626471 87.475) (end 98.6475 87.475) (width 0.2) (layer "B.Cu") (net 12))
 (segment (start 96.851471 88.25) (end 97.626471 87.475) (width 0.2) (layer "B.Cu") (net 12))
 (segment (start 98.6475 87.475) (end 98.9725 87.15) (width 0.2) (layer "B.Cu") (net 12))
 (segment (start 98.9725 87.15) (end 98.9725 86.35) (width 0.2) (layer "B.Cu") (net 12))
 (segment (start 98.235 83.192094) (end 98.235 82.515) (width 0.2) (layer "B.Cu") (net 18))
 (segment (start 99.4725 87.4725) (end 99.4725 84.429594) (width 0.2) (layer "B.Cu") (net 18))
 (segment (start 98.9725 81.7775) (end 98.9725 81.15) (width 0.2) (layer "B.Cu") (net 18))
 (segment (start 99.4725 84.429594) (end 98.235 83.192094) (width 0.2) (layer "B.Cu") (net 18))
 (segment (start 100.25 88.25) (end 99.4725 87.4725) (width 0.2) (layer "B.Cu") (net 18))
 (segment (start 98.235 82.515) (end 98.9725 81.7775) (width 0.2) (layer "B.Cu") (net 18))
 (segment (start 93.275 79.775) (end 92.3625 79.775) (width 0.2) (layer "B.Cu") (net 13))
 (segment (start 92.3625 79.775) (end 91.5875 79) (width 0.2) (layer "B.Cu") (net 13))
 (segment (start 91.5875 79) (end 91.425 79) (width 0.2) (layer "B.Cu") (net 13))
 (segment (start 94.5275 81.15) (end 94.5275 81.0275) (width 0.2) (layer "B.Cu") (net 13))
 (segment (start 94.5275 81.0275) (end 93.275 79.775) (width 0.2) (layer "B.Cu") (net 13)))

